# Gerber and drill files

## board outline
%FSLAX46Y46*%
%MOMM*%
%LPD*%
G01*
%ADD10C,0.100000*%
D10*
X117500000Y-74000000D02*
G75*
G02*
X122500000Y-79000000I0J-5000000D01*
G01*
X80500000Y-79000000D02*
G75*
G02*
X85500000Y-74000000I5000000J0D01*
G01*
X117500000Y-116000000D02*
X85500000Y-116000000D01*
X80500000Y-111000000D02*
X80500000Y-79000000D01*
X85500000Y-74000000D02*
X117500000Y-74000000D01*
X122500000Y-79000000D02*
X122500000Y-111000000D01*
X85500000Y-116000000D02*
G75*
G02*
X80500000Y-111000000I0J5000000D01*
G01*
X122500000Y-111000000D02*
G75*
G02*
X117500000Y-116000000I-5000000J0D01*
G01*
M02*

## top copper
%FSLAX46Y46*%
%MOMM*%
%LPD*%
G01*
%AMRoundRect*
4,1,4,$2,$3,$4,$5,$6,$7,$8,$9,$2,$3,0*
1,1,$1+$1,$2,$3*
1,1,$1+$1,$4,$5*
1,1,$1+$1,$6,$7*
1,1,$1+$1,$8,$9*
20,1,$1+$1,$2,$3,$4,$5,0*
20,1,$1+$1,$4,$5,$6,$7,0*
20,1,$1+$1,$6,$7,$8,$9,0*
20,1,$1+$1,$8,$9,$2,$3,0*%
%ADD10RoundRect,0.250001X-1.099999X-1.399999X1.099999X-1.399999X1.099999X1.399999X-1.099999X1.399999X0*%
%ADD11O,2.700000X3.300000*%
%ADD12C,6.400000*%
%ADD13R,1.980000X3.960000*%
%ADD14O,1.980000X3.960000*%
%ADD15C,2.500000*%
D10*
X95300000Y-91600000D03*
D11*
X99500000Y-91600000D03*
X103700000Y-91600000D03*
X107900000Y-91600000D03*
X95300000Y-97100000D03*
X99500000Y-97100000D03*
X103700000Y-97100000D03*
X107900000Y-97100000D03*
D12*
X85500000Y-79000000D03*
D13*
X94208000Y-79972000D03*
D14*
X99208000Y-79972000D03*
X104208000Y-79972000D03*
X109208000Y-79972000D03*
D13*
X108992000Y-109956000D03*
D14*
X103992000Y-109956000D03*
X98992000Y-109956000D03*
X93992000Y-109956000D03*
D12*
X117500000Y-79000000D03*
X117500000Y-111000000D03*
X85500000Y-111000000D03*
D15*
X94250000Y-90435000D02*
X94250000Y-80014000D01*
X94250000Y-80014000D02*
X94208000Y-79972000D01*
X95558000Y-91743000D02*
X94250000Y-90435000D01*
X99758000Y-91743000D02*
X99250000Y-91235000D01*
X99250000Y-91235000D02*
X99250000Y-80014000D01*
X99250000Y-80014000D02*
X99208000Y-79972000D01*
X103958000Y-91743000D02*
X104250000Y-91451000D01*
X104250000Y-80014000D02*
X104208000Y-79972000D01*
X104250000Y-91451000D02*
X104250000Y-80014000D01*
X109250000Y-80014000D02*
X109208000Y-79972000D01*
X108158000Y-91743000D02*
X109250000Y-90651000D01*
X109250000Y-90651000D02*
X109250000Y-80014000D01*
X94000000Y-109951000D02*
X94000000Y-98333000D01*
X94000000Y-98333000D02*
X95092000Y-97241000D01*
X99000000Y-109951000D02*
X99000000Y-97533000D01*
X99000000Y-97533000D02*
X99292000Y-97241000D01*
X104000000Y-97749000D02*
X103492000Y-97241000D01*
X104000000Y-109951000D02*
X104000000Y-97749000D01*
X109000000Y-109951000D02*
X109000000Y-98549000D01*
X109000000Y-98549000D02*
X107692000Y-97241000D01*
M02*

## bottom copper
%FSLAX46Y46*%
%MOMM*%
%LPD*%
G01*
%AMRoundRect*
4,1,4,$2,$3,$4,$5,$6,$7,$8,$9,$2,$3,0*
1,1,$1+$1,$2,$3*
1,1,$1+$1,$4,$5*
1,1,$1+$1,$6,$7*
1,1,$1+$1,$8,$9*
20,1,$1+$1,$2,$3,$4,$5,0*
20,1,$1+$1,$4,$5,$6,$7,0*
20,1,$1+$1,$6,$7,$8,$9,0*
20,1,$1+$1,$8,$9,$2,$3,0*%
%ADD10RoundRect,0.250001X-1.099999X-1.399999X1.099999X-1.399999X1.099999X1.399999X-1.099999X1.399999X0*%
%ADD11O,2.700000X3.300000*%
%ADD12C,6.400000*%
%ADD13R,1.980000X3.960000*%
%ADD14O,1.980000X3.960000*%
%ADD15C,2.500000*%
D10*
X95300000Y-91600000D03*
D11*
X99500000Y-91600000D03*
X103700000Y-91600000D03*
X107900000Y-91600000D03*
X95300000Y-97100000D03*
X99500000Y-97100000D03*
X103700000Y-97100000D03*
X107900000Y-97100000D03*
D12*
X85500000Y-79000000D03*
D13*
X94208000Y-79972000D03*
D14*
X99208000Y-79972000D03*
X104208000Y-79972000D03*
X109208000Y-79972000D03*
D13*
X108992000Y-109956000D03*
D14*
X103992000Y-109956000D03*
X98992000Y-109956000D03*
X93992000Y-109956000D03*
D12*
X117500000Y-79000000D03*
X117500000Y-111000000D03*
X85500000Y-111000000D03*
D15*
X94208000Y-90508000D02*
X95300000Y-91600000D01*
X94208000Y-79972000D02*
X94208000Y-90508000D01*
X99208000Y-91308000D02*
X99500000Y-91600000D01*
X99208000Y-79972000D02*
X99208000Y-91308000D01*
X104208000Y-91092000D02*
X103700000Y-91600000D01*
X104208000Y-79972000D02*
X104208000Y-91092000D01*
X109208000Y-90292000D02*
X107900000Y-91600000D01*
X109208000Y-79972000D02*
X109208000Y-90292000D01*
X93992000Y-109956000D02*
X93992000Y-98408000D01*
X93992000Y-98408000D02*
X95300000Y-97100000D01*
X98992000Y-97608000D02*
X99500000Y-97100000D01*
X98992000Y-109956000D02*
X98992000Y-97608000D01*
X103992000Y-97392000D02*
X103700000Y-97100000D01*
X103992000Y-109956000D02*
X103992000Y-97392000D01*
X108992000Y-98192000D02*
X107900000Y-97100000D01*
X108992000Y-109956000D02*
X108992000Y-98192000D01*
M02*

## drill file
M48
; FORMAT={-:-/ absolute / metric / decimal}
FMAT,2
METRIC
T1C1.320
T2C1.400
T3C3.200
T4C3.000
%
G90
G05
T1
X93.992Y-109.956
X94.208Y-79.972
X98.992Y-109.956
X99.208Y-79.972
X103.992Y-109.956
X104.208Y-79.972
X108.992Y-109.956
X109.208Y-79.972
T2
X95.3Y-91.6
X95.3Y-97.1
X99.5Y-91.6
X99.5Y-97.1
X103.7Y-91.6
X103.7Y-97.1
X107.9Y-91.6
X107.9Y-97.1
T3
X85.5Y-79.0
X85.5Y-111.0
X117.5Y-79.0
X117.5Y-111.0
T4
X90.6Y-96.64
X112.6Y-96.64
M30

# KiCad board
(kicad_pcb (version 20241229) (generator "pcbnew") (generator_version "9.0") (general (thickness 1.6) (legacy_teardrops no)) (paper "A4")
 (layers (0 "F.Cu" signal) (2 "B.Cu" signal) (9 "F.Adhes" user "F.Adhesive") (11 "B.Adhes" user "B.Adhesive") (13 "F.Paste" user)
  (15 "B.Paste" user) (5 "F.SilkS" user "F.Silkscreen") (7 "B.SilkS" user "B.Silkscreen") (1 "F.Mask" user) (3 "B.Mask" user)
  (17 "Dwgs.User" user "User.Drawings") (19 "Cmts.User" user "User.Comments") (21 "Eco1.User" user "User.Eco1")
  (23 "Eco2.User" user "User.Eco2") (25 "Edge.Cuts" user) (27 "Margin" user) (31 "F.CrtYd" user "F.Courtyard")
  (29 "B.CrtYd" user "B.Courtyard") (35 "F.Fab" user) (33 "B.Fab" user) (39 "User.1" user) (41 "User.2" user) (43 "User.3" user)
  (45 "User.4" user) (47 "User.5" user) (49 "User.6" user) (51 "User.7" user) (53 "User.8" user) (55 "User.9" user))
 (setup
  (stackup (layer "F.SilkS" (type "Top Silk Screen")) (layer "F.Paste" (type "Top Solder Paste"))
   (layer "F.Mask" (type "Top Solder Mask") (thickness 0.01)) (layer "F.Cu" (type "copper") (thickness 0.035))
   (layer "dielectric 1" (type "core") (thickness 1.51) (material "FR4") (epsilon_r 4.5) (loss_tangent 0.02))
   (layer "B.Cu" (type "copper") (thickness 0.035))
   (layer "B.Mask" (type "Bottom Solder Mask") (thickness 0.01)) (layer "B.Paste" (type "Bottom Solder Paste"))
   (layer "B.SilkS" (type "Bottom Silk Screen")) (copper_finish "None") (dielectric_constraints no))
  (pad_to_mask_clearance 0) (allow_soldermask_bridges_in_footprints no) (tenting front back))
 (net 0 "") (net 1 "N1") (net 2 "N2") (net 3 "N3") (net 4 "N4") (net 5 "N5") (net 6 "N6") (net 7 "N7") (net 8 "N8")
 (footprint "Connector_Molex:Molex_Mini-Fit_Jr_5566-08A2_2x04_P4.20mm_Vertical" (layer "F.Cu") (at 95.3 91.6)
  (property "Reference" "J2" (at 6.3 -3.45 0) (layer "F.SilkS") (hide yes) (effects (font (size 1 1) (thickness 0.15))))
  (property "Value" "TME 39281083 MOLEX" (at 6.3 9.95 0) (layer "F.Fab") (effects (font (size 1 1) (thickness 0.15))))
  (pad "" np_thru_hole circle (at -4.7 5.04) (size 3 3) (drill 3) (layers "*.Cu" "*.Mask"))
  (pad "" np_thru_hole circle (at 17.3 5.04) (size 3 3) (drill 3) (layers "*.Cu" "*.Mask"))
  (pad "1" thru_hole roundrect (at 0 0) (size 2.7 3.3) (drill 1.4) (layers "*.Cu" "*.Mask") (remove_unused_layers no)
   (roundrect_rratio 0.092593) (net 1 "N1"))
  (pad "2" thru_hole oval (at 4.2 0) (size 2.7 3.3) (drill 1.4) (layers "*.Cu" "*.Mask") (remove_unused_layers no) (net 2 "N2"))
  (pad "3" thru_hole oval (at 8.4 0) (size 2.7 3.3) (drill 1.4) (layers "*.Cu" "*.Mask") (remove_unused_layers no) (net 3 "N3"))
  (pad "4" thru_hole oval (at 12.6 0) (size 2.7 3.3) (drill 1.4) (layers "*.Cu" "*.Mask") (remove_unused_layers no) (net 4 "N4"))
  (pad "5" thru_hole oval (at 0 5.5) (size 2.7 3.3) (drill 1.4) (layers "*.Cu" "*.Mask") (remove_unused_layers no) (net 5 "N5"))
  (pad "6" thru_hole oval (at 4.2 5.5) (size 2.7 3.3) (drill 1.4) (layers "*.Cu" "*.Mask") (remove_unused_layers no) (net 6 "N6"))
  (pad "7" thru_hole oval (at 8.4 5.5) (size 2.7 3.3) (drill 1.4) (layers "*.Cu" "*.Mask") (remove_unused_layers no) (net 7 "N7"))
  (pad "8" thru_hole oval (at 12.6 5.5) (size 2.7 3.3) (drill 1.4) (layers "*.Cu" "*.Mask") (remove_unused_layers no) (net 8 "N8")))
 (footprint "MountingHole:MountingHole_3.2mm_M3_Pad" (layer "F.Cu") (at 85.5 79)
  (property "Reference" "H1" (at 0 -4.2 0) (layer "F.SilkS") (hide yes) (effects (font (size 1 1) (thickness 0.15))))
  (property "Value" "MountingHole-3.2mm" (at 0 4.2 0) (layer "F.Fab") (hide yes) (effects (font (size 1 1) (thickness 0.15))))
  (pad "1" thru_hole circle (at 0 0) (size 6.4 6.4) (drill 3.2) (layers "*.Cu" "*.Mask") (remove_unused_layers no)))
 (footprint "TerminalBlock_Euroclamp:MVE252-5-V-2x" (layer "F.Cu") (at 101.6 80.2)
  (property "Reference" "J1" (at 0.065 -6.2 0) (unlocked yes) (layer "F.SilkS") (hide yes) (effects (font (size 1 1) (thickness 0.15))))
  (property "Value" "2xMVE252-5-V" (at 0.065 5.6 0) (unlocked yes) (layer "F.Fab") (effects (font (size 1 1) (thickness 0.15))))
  (pad "1" thru_hole rect (at -7.392 -0.228) (size 1.98 3.96) (drill 1.32) (layers "*.Cu" "*.Mask") (remove_unused_layers no) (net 1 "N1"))
  (pad "2" thru_hole oval (at -2.392 -0.228) (size 1.98 3.96) (drill 1.32) (layers "*.Cu" "*.Mask") (remove_unused_layers no) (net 2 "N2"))
  (pad "3" thru_hole oval (at 2.608 -0.228) (size 1.98 3.96) (drill 1.32) (layers "*.Cu" "*.Mask") (remove_unused_layers no) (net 3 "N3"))
  (pad "4" thru_hole oval (at 7.608 -0.228) (size 1.98 3.96) (drill 1.32) (layers "*.Cu" "*.Mask") (remove_unused_layers no) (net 4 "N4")))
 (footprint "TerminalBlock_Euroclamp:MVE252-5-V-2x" (layer "F.Cu") (at 101.6 109.728 180)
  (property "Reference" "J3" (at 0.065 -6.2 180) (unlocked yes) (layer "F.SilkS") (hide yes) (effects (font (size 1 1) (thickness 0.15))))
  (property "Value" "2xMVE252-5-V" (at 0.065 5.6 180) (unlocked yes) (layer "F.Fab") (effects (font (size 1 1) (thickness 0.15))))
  (pad "1" thru_hole rect (at -7.392 -0.228 180) (size 1.98 3.96) (drill 1.32) (layers "*.Cu" "*.Mask") (remove_unused_layers no)
   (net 8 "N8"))
  (pad "2" thru_hole oval (at -2.392 -0.228 180) (size 1.98 3.96) (drill 1.32) (layers "*.Cu" "*.Mask") (remove_unused_layers no)
   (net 7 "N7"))
  (pad "3" thru_hole oval (at 2.608 -0.228 180) (size 1.98 3.96) (drill 1.32) (layers "*.Cu" "*.Mask") (remove_unused_layers no)
   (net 6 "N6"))
  (pad "4" thru_hole oval (at 7.608 -0.228 180) (size 1.98 3.96) (drill 1.32) (layers "*.Cu" "*.Mask") (remove_unused_layers no)
   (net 5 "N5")))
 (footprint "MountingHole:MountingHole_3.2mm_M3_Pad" (layer "F.Cu") (at 117.5 79)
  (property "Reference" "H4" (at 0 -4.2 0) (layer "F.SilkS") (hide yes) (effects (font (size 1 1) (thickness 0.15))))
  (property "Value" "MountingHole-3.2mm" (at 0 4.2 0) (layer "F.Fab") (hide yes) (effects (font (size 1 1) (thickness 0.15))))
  (pad "1" thru_hole circle (at 0 0) (size 6.4 6.4) (drill 3.2) (layers "*.Cu" "*.Mask") (remove_unused_layers no)))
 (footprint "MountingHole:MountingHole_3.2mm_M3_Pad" (layer "F.Cu") (at 117.5 111)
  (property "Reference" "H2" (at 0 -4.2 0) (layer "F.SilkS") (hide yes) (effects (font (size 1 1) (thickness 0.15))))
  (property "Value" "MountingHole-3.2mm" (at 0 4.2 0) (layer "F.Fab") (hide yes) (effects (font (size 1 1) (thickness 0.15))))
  (pad "1" thru_hole circle (at 0 0) (size 6.4 6.4) (drill 3.2) (layers "*.Cu" "*.Mask") (remove_unused_layers no)))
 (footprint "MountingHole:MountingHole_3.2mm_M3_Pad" (layer "F.Cu") (at 85.5 111)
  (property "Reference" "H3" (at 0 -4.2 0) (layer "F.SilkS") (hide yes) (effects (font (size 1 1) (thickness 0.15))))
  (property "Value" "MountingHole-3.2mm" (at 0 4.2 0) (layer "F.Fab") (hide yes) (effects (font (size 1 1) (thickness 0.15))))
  (pad "1" thru_hole circle (at 0 0) (size 6.4 6.4) (drill 3.2) (layers "*.Cu" "*.Mask") (remove_unused_layers no)))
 (gr_arc (start 117.5 74) (mid 121.035534 75.464466) (end 122.5 79) (stroke (width 0.1) (type solid)) (layer "Edge.Cuts"))
 (gr_arc (start 80.5 79) (mid 81.964466 75.464466) (end 85.5 74) (stroke (width 0.1) (type solid)) (layer "Edge.Cuts"))
 (gr_line (start 117.5 116) (end 85.5 116) (stroke (width 0.1) (type solid)) (layer "Edge.Cuts"))
 (gr_line (start 80.5 111) (end 80.5 79) (stroke (width 0.1) (type solid)) (layer "Edge.Cuts"))
 (gr_line (start 85.5 74) (end 117.5 74) (stroke (width 0.1) (type solid)) (layer "Edge.Cuts"))
 (gr_line (start 122.5 79) (end 122.5 111) (stroke (width 0.1) (type solid)) (layer "Edge.Cuts"))
 (gr_arc (start 85.5 116) (mid 81.964466 114.535534) (end 80.5 111) (stroke (width 0.1) (type solid)) (layer "Edge.Cuts"))
 (gr_arc (start 122.5 111) (mid 121.035534 114.535534) (end 117.5 116) (stroke (width 0.1) (type solid)) (layer "Edge.Cuts"))
 (segment (start 94.25 90.435) (end 94.25 80.014) (width 2.5) (layer "F.Cu") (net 1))
 (segment (start 94.25 80.014) (end 94.208 79.972) (width 2.5) (layer "F.Cu") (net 1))
 (segment (start 95.558 91.743) (end 94.25 90.435) (width 2.5) (layer "F.Cu") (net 1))
 (segment (start 94.208 90.508) (end 95.3 91.6) (width 2.5) (layer "B.Cu") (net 1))
 (segment (start 94.208 79.972) (end 94.208 90.508) (width 2.5) (layer "B.Cu") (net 1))
 (segment (start 99.758 91.743) (end 99.25 91.235) (width 2.5) (layer "F.Cu") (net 2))
 (segment (start 99.25 91.235) (end 99.25 80.014) (width 2.5) (layer "F.Cu") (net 2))
 (segment (start 99.25 80.014) (end 99.208 79.972) (width 2.5) (layer "F.Cu") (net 2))
 (segment (start 99.208 91.308) (end 99.5 91.6) (width 2.5) (layer "B.Cu") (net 2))
 (segment (start 99.208 79.972) (end 99.208 91.308) (width 2.5) (layer "B.Cu") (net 2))
 (segment (start 103.958 91.743) (end 104.25 91.451) (width 2.5) (layer "F.Cu") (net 3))
 (segment (start 104.25 80.014) (end 104.208 79.972) (width 2.5) (layer "F.Cu") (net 3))
 (segment (start 104.25 91.451) (end 104.25 80.014) (width 2.5) (layer "F.Cu") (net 3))
 (segment (start 104.208 91.092) (end 103.7 91.6) (width 2.5) (layer "B.Cu") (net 3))
 (segment (start 104.208 79.972) (end 104.208 91.092) (width 2.5) (layer "B.Cu") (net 3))
 (segment (start 109.25 80.014) (end 109.208 79.972) (width 2.5) (layer "F.Cu") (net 4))
 (segment (start 108.158 91.743) (end 109.25 90.651) (width 2.5) (layer "F.Cu") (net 4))
 (segment (start 109.25 90.651) (end 109.25 80.014) (width 2.5) (layer "F.Cu") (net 4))
 (segment (start 109.208 90.292) (end 107.9 91.6) (width 2.5) (layer "B.Cu") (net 4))
 (segment (start 109.208 79.972) (end 109.208 90.292) (width 2.5) (layer "B.Cu") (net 4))
 (segment (start 94 109.951) (end 94 98.333) (width 2.5) (layer "F.Cu") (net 5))
 (segment (start 94 98.333) (end 95.092 97.241) (width 2.5) (layer "F.Cu") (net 5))
 (segment (start 93.992 109.956) (end 93.992 98.408) (width 2.5) (layer "B.Cu") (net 5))
 (segment (start 93.992 98.408) (end 95.3 97.1) (width 2.5) (layer "B.Cu") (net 5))
 (segment (start 99 109.951) (end 99 97.533) (width 2.5) (layer "F.Cu") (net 6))
 (segment (start 99 97.533) (end 99.292 97.241) (width 2.5) (layer "F.Cu") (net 6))
 (segment (start 98.992 97.608) (end 99.5 97.1) (width 2.5) (layer "B.Cu") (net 6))
 (segment (start 98.992 109.956) (end 98.992 97.608) (width 2.5) (layer "B.Cu") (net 6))
 (segment (start 104 97.749) (end 103.492 97.241) (width 2.5) (layer "F.Cu") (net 7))
 (segment (start 104 109.951) (end 104 97.749) (width 2.5) (layer "F.Cu") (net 7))
 (segment (start 103.992 97.392) (end 103.7 97.1) (width 2.5) (layer "B.Cu") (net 7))
 (segment (start 103.992 109.956) (end 103.992 97.392) (width 2.5) (layer "B.Cu") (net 7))
 (segment (start 109 109.951) (end 109 98.549) (width 2.5) (layer "F.Cu") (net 8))
 (segment (start 109 98.549) (end 107.692 97.241) (width 2.5) (layer "F.Cu") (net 8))
 (segment (start 108.992 98.192) (end 107.9 97.1) (width 2.5) (layer "B.Cu") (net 8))
 (segment (start 108.992 109.956) (end 108.992 98.192) (width 2.5) (layer "B.Cu") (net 8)))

